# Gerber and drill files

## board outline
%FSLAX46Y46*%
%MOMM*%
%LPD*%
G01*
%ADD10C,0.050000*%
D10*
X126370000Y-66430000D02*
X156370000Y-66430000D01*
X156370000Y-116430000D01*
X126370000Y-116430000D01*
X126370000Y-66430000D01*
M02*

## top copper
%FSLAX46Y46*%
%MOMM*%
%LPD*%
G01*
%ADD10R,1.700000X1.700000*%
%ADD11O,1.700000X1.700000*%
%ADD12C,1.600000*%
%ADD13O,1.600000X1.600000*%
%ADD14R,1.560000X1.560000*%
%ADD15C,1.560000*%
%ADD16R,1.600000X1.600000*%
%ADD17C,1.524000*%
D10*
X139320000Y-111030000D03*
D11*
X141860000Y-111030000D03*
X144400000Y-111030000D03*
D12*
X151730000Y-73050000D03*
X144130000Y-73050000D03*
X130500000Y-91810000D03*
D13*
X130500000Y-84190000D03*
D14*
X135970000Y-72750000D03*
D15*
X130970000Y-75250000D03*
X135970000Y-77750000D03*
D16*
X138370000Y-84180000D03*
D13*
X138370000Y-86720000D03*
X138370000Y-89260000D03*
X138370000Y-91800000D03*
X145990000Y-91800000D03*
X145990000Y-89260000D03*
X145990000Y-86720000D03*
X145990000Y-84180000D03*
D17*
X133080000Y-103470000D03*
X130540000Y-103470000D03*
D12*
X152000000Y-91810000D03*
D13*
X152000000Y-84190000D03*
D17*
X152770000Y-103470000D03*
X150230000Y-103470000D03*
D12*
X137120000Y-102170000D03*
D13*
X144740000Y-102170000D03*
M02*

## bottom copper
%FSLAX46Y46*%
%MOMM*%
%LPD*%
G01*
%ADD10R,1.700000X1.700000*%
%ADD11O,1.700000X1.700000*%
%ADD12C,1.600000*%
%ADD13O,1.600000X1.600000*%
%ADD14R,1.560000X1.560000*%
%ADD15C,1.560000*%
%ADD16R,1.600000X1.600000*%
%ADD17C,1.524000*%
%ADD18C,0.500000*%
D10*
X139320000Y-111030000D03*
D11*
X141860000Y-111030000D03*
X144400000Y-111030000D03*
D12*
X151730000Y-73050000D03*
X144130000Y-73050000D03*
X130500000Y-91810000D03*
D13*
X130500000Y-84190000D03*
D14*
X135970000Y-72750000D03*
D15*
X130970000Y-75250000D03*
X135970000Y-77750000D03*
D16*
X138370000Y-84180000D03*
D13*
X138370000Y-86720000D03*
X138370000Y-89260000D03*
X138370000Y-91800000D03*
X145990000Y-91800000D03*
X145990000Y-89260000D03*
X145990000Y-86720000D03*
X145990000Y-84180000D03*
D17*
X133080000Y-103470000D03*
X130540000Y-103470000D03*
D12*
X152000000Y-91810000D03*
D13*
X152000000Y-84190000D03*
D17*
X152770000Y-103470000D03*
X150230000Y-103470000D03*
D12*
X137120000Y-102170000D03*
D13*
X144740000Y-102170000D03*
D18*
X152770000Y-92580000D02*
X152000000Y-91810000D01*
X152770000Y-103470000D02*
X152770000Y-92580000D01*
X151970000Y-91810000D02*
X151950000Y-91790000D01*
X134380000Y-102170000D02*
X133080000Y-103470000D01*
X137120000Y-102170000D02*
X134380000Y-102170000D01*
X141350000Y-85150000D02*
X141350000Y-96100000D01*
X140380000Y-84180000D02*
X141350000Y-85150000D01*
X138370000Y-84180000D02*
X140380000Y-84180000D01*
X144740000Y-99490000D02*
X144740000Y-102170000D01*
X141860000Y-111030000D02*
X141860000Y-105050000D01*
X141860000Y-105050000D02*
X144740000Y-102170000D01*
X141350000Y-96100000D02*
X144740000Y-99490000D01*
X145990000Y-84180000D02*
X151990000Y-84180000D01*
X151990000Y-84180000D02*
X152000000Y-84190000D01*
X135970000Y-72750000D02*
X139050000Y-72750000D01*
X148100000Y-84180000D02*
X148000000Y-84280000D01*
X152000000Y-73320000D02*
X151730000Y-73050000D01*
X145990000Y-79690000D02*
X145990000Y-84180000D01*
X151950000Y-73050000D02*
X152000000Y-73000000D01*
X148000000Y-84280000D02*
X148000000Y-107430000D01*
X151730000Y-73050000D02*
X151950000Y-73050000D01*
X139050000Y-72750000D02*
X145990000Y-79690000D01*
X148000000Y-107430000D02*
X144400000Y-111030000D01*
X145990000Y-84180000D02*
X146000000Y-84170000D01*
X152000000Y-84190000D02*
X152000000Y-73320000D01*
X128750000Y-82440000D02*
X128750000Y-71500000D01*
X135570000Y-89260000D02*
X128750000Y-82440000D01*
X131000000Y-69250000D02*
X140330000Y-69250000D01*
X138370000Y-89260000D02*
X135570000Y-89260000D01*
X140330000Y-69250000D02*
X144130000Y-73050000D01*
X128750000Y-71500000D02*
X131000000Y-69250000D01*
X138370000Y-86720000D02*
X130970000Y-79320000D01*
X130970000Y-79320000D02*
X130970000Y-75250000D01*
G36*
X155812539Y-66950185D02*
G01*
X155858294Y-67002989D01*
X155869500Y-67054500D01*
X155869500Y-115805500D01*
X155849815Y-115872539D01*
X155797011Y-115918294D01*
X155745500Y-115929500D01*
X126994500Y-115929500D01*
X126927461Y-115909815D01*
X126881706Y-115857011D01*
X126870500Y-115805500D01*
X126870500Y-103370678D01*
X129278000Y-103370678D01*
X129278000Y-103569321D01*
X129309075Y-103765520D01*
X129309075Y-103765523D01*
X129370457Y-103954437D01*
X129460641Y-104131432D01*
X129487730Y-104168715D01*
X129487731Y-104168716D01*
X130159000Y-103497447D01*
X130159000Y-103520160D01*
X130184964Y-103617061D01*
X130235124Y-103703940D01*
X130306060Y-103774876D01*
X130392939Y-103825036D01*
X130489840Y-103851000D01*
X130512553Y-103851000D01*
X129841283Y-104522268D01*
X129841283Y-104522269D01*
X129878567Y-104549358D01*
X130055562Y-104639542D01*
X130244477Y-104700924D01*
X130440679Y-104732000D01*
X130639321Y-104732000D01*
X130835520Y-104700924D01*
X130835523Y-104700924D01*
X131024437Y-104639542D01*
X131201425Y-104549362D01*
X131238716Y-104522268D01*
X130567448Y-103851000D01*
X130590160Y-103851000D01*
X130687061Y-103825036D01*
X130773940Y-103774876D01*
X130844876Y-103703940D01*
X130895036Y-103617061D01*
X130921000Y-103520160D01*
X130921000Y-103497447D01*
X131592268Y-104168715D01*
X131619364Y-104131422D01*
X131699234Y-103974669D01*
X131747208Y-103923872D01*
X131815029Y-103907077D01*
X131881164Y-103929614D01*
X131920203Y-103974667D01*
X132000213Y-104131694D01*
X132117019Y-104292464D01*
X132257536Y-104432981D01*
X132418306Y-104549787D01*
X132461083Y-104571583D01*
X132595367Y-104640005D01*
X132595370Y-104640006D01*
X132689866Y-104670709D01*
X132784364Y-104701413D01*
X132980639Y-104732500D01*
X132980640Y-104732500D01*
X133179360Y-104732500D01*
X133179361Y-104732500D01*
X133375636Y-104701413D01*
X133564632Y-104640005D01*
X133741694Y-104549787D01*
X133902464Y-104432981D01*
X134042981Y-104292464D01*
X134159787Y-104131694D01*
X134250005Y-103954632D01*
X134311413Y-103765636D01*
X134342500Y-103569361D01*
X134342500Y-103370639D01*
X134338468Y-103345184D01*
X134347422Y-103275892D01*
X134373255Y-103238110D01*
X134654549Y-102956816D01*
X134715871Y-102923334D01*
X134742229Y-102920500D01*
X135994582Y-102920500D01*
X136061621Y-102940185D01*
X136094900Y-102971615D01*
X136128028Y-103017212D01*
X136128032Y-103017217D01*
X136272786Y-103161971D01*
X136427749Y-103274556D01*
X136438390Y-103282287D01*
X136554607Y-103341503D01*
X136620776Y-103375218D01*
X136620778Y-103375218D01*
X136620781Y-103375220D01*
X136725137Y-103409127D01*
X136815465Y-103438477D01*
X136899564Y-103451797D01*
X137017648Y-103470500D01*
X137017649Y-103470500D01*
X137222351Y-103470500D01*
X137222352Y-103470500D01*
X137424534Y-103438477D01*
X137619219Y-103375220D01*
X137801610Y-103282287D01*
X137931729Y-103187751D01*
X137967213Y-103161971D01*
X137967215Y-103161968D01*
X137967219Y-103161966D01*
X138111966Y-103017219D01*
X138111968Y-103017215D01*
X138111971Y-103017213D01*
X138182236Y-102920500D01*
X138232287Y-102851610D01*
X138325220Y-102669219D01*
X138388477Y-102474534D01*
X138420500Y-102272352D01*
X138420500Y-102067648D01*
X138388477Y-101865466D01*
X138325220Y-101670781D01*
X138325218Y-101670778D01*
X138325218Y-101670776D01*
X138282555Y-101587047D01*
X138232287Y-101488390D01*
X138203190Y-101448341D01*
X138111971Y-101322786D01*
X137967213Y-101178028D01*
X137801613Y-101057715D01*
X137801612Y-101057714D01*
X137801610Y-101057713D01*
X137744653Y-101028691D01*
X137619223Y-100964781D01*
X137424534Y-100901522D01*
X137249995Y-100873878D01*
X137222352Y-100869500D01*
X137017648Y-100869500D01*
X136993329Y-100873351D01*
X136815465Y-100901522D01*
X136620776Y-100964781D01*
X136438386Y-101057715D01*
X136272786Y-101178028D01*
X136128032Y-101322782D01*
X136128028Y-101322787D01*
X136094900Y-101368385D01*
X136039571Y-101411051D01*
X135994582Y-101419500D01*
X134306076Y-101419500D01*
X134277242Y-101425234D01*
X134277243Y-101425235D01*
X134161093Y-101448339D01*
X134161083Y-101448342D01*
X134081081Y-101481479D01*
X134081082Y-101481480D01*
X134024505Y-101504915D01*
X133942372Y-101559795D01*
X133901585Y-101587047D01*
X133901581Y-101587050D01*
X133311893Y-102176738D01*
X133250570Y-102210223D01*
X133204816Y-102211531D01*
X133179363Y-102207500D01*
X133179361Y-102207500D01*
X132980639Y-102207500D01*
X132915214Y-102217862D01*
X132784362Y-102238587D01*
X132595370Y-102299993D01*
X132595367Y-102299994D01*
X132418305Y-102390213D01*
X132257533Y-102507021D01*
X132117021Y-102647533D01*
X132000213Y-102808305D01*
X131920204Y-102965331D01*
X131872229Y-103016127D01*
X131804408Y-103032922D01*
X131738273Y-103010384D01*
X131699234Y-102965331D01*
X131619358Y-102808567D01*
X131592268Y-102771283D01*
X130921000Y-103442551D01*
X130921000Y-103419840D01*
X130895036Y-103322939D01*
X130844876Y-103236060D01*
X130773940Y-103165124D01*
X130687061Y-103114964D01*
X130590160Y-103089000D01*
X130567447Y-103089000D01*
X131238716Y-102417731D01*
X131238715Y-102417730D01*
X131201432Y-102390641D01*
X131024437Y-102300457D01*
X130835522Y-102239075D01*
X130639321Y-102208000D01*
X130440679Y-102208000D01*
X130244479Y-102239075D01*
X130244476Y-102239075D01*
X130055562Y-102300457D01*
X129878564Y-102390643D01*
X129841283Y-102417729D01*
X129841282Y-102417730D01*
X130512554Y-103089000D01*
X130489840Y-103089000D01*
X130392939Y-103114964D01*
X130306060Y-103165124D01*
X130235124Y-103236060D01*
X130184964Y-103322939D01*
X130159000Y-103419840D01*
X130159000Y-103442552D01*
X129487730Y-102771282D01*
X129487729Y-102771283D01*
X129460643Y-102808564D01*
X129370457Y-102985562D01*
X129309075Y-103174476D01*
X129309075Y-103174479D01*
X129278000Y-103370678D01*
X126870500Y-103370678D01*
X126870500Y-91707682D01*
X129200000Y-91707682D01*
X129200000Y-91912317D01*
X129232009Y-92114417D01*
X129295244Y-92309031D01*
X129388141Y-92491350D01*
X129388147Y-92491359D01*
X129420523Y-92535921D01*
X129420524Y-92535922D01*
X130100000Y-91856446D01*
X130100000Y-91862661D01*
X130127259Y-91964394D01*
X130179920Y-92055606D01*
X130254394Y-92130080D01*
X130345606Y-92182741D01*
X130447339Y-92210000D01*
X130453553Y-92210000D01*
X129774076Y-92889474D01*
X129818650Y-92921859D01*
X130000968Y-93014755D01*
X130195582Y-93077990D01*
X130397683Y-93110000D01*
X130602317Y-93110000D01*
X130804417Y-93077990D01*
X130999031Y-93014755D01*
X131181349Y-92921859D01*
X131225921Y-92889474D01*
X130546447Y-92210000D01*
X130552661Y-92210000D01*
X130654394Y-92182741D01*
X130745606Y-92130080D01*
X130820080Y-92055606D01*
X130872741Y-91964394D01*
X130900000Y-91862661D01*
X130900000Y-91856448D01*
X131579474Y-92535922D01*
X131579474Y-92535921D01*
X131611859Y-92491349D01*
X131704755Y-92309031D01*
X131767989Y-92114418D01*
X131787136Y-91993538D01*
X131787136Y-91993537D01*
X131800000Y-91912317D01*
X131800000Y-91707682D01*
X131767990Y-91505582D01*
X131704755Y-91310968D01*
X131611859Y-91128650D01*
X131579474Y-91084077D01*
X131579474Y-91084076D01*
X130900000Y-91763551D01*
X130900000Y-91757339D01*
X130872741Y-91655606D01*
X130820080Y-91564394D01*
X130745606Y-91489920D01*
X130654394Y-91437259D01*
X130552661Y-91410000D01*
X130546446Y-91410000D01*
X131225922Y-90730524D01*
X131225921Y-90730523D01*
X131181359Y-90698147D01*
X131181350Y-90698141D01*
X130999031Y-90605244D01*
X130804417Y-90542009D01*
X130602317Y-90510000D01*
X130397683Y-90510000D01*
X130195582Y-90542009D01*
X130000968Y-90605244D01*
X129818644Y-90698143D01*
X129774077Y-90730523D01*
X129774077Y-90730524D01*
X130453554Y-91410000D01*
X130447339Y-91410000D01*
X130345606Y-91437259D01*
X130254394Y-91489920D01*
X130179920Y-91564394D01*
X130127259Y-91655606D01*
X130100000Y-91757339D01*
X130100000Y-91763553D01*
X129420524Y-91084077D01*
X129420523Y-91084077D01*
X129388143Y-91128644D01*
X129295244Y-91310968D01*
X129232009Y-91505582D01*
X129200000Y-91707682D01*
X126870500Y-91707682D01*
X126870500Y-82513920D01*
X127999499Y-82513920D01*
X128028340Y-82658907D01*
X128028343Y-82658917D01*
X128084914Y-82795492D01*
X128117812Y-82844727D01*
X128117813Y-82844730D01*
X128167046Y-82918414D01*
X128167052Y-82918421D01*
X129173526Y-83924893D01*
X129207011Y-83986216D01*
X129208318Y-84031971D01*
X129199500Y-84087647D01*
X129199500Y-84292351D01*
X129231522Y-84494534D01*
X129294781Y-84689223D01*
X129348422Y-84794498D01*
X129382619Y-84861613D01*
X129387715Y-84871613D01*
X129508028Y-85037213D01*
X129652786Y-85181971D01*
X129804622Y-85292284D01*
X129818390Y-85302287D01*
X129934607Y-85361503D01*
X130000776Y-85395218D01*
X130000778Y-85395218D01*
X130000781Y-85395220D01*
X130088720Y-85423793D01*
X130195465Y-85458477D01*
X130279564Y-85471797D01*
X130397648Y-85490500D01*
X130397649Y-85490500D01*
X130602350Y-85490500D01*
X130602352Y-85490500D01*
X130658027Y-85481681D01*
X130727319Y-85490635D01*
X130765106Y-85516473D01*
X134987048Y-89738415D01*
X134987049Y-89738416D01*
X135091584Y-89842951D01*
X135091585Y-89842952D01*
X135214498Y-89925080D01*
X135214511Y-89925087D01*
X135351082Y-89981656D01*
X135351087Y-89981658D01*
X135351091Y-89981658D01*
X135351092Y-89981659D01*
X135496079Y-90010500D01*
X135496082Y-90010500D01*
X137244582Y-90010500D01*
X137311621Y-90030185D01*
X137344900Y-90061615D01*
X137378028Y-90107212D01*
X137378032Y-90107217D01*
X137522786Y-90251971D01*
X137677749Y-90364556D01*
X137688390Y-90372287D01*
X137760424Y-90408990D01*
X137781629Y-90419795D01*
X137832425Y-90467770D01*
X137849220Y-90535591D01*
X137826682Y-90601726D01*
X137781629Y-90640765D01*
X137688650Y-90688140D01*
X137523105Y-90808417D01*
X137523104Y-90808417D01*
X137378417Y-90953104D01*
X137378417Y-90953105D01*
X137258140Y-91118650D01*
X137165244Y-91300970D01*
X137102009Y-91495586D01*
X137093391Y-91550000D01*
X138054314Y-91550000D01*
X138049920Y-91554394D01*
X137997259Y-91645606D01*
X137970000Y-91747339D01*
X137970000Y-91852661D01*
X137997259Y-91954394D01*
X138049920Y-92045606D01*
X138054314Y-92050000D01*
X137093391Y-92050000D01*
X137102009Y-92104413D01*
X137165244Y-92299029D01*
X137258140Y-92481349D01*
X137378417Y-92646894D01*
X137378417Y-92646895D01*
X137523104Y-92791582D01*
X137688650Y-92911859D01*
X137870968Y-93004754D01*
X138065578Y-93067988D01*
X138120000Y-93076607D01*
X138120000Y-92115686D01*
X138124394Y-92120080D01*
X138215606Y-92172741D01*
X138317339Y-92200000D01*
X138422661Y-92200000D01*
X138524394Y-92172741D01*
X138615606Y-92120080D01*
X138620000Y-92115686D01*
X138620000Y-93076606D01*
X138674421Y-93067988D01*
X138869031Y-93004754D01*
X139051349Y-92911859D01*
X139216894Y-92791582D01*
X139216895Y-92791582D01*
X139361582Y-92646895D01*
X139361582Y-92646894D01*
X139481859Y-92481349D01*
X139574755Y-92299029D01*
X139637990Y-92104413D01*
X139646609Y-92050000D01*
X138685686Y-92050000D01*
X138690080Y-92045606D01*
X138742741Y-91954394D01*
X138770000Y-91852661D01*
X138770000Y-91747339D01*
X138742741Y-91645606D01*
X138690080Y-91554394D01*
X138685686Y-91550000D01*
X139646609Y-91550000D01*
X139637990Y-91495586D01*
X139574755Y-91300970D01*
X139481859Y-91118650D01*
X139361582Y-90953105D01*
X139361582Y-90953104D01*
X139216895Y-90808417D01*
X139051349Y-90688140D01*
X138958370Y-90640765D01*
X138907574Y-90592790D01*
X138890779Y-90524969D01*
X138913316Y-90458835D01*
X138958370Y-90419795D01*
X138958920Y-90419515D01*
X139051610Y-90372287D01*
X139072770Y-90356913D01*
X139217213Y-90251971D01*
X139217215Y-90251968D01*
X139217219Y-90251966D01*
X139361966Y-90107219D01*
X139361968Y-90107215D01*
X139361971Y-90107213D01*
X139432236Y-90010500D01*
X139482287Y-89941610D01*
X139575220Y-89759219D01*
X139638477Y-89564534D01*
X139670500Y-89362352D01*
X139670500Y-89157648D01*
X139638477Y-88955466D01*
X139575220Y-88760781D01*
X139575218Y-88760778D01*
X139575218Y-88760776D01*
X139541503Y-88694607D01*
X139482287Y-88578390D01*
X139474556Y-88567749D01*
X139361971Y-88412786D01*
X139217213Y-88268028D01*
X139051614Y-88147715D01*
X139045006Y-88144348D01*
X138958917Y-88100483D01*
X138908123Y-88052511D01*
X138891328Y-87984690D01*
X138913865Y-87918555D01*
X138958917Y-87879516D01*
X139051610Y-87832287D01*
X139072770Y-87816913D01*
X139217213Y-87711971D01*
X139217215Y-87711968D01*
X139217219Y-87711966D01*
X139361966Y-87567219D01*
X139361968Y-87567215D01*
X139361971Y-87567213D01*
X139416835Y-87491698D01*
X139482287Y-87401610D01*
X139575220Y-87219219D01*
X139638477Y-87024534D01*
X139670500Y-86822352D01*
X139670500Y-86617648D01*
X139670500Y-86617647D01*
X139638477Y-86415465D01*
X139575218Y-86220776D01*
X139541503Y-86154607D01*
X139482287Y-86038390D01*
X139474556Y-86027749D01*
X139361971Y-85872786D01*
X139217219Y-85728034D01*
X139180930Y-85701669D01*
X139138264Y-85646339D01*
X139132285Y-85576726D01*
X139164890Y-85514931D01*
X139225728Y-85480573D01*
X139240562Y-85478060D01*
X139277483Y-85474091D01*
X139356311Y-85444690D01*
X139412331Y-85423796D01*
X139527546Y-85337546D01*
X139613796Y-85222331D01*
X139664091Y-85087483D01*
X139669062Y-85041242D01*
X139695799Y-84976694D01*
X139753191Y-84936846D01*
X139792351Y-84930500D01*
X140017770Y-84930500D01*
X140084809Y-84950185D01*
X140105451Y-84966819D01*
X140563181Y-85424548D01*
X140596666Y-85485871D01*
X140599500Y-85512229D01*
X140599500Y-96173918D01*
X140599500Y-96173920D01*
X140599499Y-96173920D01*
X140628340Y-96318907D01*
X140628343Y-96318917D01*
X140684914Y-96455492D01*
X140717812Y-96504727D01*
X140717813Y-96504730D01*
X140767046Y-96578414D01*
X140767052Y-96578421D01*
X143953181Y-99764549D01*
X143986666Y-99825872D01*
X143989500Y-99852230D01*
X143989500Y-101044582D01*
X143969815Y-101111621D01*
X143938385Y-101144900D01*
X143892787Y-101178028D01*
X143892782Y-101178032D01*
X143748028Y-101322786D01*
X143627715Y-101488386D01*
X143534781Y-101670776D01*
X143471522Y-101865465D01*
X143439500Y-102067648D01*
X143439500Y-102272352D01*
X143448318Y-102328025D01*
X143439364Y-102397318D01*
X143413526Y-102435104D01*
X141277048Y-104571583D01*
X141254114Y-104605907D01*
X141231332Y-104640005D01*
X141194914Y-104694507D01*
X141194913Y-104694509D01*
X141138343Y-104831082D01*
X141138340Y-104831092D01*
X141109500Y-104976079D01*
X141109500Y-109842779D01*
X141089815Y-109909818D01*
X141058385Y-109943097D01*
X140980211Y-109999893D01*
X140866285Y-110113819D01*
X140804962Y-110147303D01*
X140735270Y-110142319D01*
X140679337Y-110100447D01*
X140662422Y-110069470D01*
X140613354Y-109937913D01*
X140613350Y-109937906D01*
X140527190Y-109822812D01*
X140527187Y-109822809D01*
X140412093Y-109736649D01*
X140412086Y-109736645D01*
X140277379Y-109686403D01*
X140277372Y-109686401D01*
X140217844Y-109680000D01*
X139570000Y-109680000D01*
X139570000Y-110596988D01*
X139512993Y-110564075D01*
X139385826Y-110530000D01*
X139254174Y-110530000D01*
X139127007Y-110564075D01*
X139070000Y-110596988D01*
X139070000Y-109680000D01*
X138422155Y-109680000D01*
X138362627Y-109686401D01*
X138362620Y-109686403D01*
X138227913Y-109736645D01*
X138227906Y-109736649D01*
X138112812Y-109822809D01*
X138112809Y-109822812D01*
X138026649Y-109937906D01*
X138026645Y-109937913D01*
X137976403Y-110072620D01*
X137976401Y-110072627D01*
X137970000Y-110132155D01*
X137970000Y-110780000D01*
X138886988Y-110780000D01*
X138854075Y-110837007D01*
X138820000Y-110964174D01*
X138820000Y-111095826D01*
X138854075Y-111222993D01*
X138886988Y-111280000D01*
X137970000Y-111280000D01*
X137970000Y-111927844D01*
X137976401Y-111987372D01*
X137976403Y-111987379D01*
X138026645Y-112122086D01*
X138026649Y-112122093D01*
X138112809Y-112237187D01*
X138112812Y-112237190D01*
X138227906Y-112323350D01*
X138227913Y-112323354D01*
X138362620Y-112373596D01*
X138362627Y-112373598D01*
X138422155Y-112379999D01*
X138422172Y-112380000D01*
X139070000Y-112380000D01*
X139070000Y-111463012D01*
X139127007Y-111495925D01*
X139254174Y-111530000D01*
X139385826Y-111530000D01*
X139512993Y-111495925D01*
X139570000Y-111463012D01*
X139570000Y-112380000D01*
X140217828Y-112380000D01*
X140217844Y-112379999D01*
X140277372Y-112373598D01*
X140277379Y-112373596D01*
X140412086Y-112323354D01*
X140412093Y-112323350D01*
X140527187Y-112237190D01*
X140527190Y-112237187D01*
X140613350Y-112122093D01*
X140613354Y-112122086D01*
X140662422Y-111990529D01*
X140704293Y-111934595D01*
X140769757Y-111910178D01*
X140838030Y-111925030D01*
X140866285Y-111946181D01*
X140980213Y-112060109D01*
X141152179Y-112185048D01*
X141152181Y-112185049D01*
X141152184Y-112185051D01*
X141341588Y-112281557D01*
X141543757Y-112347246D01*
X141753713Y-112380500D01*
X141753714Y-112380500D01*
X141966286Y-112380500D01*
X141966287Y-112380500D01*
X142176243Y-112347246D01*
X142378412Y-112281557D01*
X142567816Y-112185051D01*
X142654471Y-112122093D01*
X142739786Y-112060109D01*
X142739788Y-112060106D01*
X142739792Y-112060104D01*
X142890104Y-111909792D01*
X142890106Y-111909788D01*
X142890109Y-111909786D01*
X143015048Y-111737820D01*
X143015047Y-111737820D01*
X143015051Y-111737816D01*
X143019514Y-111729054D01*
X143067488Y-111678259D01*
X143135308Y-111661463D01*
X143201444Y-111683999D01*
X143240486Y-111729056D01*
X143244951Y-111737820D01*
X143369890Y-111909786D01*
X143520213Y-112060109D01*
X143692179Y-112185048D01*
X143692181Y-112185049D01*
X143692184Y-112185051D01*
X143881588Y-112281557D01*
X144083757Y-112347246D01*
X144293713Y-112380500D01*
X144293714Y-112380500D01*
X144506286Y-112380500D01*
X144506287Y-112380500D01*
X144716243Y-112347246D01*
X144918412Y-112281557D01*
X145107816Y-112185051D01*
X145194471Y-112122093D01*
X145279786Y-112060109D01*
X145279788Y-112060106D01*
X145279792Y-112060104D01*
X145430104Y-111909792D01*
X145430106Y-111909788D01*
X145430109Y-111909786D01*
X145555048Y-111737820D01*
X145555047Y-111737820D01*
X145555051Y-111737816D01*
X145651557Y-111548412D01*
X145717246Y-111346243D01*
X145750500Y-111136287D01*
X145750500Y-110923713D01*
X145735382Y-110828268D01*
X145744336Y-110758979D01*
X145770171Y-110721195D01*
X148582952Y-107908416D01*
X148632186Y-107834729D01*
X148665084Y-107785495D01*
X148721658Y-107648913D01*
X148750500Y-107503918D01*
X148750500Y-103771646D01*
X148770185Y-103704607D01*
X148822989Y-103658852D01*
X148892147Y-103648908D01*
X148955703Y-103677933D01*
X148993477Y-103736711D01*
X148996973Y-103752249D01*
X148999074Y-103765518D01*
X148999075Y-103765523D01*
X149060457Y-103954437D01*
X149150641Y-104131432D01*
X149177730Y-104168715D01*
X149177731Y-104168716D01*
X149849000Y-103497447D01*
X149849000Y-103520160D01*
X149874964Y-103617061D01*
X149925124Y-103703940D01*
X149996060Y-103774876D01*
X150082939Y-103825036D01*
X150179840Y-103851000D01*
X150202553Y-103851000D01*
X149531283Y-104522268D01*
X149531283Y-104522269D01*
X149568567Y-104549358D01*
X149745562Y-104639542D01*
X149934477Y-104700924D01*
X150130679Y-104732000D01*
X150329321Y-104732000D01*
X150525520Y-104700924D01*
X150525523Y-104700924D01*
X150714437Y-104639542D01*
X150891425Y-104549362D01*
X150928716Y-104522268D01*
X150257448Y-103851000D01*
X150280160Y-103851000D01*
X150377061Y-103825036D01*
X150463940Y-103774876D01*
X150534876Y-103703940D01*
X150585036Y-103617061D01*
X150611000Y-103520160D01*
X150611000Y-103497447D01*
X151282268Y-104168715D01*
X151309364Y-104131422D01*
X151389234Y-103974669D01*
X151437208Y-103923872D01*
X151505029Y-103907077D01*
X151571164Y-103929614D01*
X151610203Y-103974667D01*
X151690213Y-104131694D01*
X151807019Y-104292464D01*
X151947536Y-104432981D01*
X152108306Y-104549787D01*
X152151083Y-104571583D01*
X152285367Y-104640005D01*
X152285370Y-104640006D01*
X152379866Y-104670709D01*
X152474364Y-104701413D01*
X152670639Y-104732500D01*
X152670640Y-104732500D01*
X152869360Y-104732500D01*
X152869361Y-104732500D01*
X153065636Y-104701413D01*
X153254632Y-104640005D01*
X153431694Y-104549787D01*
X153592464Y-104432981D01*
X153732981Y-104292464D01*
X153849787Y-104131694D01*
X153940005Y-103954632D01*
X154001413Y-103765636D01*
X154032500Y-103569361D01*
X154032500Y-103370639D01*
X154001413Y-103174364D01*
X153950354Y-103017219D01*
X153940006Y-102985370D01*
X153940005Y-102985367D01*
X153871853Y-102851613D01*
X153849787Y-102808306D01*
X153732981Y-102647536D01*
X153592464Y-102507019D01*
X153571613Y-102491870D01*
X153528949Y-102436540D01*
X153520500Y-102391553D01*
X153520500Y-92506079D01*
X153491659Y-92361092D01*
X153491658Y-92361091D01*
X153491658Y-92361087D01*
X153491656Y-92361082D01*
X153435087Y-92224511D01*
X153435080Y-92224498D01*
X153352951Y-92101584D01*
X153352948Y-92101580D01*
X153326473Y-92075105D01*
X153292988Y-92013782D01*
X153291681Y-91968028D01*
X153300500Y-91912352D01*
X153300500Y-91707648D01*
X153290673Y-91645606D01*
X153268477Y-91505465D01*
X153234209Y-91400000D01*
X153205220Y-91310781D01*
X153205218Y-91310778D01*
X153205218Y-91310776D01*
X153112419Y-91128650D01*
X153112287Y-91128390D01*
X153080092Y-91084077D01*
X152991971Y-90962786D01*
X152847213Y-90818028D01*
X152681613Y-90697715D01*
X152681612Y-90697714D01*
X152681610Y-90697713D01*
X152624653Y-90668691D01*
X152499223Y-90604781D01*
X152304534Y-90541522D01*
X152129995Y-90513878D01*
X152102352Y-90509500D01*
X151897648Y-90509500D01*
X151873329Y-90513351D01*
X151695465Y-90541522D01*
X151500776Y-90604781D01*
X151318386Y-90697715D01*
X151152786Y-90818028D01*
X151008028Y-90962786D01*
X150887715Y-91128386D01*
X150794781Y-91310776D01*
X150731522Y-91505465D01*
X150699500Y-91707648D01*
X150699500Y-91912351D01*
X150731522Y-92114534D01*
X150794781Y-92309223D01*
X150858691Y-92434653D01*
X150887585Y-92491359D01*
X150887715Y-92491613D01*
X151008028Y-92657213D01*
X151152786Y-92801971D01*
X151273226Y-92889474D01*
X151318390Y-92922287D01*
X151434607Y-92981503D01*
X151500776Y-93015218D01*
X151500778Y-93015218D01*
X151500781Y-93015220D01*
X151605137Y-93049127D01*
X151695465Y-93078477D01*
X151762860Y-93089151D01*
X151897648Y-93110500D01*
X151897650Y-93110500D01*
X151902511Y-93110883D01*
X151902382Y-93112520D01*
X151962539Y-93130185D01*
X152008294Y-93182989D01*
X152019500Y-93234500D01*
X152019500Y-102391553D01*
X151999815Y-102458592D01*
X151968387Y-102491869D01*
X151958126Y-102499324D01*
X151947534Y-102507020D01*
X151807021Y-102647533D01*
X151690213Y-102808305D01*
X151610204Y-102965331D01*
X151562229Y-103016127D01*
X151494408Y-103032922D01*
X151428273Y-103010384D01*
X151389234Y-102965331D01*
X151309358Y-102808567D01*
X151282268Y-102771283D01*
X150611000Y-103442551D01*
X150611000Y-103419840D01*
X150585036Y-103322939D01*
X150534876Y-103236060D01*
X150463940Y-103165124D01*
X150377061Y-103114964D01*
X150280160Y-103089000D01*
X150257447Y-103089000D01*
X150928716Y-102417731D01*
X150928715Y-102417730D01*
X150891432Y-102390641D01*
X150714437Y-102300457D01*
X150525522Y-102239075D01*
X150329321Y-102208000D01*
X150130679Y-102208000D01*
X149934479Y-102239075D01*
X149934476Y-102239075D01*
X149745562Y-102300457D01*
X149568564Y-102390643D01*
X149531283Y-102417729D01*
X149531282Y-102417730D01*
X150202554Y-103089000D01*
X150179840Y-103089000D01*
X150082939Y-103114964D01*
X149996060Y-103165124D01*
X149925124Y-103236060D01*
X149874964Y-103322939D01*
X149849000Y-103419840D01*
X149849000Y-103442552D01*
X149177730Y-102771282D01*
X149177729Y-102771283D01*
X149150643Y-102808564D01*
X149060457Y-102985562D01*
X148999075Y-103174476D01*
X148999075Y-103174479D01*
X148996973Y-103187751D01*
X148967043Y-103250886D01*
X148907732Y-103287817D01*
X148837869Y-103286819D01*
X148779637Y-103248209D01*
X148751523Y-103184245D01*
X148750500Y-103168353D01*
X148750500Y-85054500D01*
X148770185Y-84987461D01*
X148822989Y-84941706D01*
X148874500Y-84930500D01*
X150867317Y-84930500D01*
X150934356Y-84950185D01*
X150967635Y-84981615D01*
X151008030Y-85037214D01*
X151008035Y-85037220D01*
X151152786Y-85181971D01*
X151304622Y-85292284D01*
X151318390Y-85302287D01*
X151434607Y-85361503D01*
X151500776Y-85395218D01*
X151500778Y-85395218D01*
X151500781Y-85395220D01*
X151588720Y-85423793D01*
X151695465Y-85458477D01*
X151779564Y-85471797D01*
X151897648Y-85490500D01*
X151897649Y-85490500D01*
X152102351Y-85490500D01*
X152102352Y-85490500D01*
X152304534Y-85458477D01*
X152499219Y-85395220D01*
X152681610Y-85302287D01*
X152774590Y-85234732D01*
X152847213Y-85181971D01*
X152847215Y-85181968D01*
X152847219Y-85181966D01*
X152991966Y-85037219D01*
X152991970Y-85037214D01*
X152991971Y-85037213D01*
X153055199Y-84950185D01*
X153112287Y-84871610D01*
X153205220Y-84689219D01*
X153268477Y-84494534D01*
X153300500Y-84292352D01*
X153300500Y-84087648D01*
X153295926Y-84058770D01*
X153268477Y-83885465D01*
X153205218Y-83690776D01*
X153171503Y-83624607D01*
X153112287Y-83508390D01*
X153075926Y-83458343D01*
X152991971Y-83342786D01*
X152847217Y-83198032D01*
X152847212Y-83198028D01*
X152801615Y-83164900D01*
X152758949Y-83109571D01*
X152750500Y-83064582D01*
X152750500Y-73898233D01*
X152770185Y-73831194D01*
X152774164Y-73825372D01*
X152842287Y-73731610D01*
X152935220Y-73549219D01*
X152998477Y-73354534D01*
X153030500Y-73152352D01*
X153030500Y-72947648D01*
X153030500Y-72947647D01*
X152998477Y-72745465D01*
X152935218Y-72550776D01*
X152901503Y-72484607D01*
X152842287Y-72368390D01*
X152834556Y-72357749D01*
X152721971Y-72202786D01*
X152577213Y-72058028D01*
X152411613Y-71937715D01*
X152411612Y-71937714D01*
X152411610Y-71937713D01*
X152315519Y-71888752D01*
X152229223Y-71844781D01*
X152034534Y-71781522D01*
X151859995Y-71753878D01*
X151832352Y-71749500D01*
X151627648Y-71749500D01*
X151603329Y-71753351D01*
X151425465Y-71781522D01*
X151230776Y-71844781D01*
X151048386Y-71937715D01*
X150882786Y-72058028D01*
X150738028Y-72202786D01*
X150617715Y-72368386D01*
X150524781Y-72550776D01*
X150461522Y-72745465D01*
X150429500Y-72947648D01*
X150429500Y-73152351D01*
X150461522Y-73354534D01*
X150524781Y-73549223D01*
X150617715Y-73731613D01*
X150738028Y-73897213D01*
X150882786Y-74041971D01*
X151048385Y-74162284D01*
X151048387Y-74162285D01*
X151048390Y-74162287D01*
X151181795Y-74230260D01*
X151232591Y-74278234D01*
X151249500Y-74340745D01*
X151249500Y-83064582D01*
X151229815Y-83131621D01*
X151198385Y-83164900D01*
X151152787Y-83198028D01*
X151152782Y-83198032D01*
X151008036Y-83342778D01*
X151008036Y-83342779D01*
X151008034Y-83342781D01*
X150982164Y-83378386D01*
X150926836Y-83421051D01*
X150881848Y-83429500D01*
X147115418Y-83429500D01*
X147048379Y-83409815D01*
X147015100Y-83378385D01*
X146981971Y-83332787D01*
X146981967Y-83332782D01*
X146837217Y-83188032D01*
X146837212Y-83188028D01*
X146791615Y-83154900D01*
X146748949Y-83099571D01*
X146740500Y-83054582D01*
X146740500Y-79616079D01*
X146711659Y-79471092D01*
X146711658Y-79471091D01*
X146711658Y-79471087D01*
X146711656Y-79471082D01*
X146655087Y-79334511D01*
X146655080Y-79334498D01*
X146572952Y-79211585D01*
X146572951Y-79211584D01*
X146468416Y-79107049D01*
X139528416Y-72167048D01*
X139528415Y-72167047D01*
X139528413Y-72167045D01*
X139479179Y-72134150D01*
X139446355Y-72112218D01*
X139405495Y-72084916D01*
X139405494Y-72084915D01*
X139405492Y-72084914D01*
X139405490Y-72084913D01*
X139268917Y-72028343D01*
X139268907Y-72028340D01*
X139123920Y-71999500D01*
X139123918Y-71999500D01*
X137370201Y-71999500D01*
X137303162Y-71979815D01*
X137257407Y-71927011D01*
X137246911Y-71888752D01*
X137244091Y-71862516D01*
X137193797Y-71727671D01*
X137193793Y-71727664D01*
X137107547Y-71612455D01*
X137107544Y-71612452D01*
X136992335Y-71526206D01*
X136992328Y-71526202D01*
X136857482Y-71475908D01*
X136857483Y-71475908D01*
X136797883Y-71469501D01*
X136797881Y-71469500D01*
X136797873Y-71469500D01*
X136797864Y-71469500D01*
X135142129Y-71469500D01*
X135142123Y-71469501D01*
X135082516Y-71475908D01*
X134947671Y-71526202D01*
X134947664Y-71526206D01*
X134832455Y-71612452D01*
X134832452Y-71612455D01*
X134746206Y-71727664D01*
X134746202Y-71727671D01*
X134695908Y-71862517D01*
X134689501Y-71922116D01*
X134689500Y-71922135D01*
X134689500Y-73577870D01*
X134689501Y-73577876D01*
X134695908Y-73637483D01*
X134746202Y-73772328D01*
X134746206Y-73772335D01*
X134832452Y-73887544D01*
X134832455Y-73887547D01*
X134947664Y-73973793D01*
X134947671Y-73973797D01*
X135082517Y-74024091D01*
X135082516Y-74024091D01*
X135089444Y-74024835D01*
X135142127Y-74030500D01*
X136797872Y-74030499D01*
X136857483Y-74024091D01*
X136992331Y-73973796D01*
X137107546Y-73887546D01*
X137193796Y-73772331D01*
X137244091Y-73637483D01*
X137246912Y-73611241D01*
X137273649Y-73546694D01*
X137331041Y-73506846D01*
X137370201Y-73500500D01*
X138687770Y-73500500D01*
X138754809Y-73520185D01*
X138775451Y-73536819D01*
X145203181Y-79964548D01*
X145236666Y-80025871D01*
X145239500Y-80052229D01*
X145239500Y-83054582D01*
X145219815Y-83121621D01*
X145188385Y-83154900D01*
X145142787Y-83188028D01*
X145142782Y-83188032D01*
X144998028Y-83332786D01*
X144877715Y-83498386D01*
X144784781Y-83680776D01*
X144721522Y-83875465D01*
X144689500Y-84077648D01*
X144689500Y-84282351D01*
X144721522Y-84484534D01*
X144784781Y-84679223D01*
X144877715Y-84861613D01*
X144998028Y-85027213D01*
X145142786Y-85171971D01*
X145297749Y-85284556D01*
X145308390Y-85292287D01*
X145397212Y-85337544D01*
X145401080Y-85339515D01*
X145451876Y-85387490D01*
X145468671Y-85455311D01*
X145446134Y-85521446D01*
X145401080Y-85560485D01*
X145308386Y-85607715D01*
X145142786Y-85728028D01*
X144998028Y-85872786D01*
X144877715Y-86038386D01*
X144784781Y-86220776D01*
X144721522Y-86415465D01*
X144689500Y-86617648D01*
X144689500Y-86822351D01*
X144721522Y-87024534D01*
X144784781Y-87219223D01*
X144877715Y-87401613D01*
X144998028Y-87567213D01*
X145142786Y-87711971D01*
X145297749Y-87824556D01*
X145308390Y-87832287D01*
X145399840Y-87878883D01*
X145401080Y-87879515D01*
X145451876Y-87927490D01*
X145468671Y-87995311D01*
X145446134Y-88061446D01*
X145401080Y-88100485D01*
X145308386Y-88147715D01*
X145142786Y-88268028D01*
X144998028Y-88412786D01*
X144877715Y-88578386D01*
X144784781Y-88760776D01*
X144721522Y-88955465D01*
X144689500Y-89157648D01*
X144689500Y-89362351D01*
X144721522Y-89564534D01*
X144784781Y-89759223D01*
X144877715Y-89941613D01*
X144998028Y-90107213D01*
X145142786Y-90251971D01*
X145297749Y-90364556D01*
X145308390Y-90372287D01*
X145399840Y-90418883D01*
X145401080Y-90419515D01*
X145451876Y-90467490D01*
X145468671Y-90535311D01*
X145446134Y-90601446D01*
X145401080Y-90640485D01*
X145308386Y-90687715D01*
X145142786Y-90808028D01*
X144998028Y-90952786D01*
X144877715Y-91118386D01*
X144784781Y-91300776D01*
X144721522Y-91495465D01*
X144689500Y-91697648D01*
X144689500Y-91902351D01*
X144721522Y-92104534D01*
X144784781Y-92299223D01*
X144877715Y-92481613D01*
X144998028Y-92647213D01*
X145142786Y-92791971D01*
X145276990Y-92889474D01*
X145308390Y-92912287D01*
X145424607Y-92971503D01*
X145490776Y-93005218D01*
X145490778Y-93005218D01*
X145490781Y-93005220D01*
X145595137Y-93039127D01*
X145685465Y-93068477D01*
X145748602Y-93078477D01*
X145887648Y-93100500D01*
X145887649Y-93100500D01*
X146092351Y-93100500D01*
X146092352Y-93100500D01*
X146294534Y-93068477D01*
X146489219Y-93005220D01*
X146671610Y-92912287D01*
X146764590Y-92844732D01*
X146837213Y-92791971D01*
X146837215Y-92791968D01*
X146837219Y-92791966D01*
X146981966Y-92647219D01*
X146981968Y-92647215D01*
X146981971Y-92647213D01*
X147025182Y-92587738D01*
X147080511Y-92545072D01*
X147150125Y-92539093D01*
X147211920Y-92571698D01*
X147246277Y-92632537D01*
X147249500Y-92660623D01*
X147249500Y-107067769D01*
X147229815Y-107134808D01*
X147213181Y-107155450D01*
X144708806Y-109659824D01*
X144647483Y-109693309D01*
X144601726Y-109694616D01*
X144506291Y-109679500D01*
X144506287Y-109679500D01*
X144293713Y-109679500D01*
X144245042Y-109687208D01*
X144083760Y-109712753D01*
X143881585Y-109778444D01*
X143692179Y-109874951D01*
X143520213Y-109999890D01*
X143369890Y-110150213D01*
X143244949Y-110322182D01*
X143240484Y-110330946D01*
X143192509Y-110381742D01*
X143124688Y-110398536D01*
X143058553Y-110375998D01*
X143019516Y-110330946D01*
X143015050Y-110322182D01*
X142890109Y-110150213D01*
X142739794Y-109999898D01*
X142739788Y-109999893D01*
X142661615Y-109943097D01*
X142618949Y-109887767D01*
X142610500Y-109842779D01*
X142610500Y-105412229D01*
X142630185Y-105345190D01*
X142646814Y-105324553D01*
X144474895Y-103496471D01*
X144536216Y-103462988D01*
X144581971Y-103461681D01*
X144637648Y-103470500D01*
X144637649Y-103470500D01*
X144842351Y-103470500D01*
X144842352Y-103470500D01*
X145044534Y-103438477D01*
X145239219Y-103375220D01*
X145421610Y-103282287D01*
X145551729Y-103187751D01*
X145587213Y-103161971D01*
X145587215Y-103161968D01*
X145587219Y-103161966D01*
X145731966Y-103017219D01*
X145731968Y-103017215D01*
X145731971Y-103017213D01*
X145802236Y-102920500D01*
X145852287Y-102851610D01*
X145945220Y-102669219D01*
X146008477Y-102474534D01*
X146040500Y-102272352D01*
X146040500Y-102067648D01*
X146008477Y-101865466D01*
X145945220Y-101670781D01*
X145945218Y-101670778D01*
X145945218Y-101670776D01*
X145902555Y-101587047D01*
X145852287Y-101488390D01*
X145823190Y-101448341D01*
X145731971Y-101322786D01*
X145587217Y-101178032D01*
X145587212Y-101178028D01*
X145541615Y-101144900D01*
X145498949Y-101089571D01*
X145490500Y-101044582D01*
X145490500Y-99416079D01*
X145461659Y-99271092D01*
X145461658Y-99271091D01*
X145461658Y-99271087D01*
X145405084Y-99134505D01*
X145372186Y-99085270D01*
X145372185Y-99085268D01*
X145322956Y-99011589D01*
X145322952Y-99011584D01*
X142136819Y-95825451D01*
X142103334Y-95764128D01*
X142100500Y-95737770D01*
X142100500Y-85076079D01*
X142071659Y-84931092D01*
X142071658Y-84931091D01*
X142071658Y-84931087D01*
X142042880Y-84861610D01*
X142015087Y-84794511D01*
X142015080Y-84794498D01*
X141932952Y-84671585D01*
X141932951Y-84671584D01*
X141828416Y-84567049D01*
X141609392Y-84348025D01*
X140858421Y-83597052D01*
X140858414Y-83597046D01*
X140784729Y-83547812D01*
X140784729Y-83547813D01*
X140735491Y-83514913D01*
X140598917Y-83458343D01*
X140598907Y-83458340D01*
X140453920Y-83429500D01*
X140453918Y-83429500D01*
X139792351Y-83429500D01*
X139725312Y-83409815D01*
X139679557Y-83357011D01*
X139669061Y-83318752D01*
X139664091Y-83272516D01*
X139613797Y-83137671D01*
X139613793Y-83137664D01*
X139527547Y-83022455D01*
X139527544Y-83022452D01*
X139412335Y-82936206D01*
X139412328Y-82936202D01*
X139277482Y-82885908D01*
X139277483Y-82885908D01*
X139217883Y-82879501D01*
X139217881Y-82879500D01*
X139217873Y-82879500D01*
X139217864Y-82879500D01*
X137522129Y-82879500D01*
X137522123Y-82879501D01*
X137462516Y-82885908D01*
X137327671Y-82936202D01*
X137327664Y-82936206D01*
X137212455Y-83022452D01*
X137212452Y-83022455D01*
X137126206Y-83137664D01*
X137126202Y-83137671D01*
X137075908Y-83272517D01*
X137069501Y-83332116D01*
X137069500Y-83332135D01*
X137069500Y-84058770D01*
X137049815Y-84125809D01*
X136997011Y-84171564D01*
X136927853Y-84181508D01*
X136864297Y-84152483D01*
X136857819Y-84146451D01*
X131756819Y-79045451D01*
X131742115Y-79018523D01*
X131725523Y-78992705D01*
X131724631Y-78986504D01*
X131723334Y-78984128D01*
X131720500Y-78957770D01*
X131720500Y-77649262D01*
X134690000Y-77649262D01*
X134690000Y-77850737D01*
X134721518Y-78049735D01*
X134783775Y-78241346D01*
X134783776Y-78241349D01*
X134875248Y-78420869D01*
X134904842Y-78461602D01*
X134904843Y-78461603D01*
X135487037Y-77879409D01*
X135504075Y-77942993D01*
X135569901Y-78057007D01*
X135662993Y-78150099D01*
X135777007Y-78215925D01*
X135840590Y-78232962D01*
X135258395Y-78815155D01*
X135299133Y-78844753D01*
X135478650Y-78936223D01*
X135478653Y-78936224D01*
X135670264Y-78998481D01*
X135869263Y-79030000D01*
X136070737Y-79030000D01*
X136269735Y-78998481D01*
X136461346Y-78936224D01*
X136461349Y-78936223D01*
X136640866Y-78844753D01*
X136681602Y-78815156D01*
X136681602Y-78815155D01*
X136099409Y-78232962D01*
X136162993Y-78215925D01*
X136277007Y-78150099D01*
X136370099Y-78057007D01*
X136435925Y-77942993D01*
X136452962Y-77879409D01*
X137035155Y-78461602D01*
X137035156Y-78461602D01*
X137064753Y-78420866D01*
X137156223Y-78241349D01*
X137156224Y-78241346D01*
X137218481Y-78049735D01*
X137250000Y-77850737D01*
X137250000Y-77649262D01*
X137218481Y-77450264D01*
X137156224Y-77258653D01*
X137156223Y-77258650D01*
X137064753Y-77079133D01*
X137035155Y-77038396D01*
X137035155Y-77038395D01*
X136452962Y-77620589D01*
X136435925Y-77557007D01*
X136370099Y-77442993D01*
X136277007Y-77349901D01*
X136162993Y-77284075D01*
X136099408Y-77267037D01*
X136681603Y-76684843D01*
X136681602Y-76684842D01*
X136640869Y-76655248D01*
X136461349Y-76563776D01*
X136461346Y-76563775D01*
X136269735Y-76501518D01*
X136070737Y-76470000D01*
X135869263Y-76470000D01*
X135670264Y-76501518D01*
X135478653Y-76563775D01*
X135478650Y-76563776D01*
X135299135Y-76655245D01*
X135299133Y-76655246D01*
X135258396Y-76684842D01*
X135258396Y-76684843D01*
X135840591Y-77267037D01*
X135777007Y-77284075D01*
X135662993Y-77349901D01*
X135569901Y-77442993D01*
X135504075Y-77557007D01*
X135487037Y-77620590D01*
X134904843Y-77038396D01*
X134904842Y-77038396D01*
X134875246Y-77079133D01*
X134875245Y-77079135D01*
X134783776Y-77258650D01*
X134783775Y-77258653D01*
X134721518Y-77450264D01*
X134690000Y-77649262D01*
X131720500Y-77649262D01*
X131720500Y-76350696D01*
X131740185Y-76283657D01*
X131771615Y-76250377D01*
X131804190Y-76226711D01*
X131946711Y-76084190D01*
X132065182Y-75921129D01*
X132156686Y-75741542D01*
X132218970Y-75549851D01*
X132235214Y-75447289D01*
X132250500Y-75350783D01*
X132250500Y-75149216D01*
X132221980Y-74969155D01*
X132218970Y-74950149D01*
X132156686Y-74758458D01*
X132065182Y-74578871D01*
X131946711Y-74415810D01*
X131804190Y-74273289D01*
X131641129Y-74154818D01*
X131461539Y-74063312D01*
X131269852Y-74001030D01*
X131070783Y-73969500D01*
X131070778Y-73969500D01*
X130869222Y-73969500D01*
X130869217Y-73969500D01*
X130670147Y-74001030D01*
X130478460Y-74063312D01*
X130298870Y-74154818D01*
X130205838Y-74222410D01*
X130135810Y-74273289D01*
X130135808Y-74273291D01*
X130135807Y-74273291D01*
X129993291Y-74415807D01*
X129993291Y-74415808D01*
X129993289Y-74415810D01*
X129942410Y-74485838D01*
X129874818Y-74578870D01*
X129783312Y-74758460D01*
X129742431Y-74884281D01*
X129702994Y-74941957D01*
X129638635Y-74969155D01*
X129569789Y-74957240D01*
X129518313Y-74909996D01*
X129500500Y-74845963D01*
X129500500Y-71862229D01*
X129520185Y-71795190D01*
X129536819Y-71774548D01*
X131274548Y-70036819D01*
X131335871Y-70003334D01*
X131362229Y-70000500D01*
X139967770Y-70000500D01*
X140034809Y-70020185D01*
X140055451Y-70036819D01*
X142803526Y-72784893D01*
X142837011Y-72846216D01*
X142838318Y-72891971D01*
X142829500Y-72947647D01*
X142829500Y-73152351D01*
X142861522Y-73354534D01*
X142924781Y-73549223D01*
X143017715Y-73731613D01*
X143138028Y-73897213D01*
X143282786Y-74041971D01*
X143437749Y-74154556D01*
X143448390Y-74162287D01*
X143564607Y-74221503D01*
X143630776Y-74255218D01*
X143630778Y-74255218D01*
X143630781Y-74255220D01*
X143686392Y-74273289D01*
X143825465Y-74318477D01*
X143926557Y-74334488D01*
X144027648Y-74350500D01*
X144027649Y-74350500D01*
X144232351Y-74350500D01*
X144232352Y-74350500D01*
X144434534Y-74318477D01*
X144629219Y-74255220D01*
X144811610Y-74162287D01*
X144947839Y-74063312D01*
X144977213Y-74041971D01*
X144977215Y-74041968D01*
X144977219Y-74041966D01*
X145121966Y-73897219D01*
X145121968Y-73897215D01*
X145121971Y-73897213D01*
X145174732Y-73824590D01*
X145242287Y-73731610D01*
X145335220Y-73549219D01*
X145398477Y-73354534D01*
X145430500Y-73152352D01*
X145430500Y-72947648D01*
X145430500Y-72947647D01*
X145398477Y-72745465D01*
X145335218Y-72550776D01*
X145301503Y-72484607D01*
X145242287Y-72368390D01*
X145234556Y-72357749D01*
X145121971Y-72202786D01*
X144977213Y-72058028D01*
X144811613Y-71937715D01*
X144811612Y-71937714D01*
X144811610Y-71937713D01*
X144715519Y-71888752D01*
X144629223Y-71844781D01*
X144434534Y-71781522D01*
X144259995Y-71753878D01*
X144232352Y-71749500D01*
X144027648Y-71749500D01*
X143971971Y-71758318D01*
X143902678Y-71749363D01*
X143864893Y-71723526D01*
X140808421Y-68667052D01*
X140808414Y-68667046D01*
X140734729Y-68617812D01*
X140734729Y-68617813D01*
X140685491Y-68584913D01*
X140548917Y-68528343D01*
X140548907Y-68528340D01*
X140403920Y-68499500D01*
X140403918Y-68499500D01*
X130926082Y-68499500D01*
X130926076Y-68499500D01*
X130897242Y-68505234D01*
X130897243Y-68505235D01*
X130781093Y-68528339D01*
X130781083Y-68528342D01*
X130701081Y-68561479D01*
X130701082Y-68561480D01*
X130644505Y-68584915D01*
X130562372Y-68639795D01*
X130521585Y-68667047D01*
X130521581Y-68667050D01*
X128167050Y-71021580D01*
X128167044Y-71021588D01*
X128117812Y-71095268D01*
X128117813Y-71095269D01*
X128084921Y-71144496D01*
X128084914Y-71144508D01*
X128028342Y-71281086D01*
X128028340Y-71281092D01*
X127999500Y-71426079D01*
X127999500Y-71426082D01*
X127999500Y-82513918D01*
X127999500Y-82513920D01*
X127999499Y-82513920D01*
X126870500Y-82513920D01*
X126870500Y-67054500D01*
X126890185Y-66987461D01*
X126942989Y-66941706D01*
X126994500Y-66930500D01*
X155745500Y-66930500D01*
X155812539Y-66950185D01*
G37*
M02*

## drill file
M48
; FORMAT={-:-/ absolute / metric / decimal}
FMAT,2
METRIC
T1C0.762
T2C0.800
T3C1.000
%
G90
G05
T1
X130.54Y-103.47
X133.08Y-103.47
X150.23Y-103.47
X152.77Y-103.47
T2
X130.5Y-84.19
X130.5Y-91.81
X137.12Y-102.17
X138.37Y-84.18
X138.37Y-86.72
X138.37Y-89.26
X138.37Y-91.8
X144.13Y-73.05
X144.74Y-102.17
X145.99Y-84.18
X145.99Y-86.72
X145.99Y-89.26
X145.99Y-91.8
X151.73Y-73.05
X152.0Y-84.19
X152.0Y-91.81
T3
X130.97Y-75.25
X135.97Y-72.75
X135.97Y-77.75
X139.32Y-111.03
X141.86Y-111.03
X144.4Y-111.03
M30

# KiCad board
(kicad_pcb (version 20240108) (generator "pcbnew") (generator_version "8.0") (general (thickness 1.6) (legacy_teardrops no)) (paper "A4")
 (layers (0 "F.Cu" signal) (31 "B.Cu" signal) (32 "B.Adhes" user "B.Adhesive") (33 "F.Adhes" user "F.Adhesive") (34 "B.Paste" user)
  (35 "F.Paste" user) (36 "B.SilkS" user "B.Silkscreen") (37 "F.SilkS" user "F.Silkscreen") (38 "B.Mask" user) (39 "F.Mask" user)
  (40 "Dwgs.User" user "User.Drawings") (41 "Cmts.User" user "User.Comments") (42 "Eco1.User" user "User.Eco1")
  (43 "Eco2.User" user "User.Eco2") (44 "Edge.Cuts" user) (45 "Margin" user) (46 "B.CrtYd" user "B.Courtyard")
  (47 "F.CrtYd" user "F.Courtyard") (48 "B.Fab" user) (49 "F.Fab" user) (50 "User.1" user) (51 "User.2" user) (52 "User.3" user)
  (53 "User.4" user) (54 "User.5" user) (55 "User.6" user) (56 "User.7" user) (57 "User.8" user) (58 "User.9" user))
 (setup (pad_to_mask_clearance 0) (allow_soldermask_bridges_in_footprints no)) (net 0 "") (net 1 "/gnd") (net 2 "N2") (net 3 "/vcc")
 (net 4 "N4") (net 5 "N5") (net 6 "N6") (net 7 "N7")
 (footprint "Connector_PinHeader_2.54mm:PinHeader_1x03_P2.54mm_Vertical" (layer "F.Cu") (at 139.32 111.03 90)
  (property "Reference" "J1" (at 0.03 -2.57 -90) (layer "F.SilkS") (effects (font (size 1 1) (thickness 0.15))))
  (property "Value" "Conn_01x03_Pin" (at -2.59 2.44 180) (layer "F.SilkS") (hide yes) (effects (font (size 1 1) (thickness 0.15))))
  (pad "1" thru_hole rect (at 0 0 90) (size 1.7 1.7) (drill 1) (layers "*.Cu" "*.Mask") (remove_unused_layers no) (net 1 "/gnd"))
  (pad "2" thru_hole oval (at 0 2.54 90) (size 1.7 1.7) (drill 1) (layers "*.Cu" "*.Mask") (remove_unused_layers no) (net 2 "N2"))
  (pad "3" thru_hole oval (at 0 5.08 90) (size 1.7 1.7) (drill 1) (layers "*.Cu" "*.Mask") (remove_unused_layers no) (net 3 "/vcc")))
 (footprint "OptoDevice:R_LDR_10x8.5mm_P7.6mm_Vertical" (layer "F.Cu") (at 151.73 73.05 180)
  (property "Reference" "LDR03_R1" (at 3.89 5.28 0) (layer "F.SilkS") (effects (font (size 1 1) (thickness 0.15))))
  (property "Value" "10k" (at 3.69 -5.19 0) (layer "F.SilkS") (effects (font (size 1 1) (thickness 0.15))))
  (pad "1" thru_hole circle (at 0 0 180) (size 1.6 1.6) (drill 0.8) (layers "*.Cu" "*.Mask") (remove_unused_layers no) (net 3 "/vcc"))
  (pad "2" thru_hole circle (at 7.6 0 180) (size 1.6 1.6) (drill 0.8) (layers "*.Cu" "*.Mask") (remove_unused_layers no) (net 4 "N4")))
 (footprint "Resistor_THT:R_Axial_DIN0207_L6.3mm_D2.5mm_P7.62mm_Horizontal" (layer "F.Cu") (at 130.5 91.81 90)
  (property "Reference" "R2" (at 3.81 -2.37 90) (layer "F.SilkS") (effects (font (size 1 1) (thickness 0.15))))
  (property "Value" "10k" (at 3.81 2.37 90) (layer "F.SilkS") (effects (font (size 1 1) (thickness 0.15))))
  (pad "1" thru_hole circle (at 0 0 90) (size 1.6 1.6) (drill 0.8) (layers "*.Cu" "*.Mask") (remove_unused_layers no) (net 1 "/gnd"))
  (pad "2" thru_hole oval (at 7.62 0 90) (size 1.6 1.6) (drill 0.8) (layers "*.Cu" "*.Mask") (remove_unused_layers no) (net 4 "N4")))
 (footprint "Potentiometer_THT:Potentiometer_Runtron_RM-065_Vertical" (layer "F.Cu") (at 135.97 72.75 -90)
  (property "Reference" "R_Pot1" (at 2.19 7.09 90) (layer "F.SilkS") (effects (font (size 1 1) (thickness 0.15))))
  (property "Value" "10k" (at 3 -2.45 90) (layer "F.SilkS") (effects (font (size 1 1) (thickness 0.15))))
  (pad "1" thru_hole rect (at 0 0 270) (size 1.56 1.56) (drill 1) (layers "*.Cu" "*.Mask") (remove_unused_layers no) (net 3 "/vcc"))
  (pad "2" thru_hole circle (at 2.5 5 270) (size 1.56 1.56) (drill 1) (layers "*.Cu" "*.Mask") (remove_unused_layers no) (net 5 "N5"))
  (pad "3" thru_hole circle (at 5 0 270) (size 1.56 1.56) (drill 1) (layers "*.Cu" "*.Mask") (remove_unused_layers no) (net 1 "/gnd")))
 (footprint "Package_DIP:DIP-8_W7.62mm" (layer "F.Cu") (at 138.37 84.18)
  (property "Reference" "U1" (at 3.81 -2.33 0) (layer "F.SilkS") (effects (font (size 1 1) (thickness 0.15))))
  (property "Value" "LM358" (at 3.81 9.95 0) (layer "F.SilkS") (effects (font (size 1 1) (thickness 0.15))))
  (pad "1" thru_hole rect (at 0 0) (size 1.6 1.6) (drill 0.8) (layers "*.Cu" "*.Mask") (remove_unused_layers no) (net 2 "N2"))
  (pad "2" thru_hole oval (at 0 2.54) (size 1.6 1.6) (drill 0.8) (layers "*.Cu" "*.Mask") (remove_unused_layers no) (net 5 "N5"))
  (pad "3" thru_hole oval (at 0 5.08) (size 1.6 1.6) (drill 0.8) (layers "*.Cu" "*.Mask") (remove_unused_layers no) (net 4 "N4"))
  (pad "4" thru_hole oval (at 0 7.62) (size 1.6 1.6) (drill 0.8) (layers "*.Cu" "*.Mask") (remove_unused_layers no) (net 1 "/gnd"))
  (pad "5" thru_hole oval (at 7.62 7.62) (size 1.6 1.6) (drill 0.8) (layers "*.Cu" "*.Mask") (remove_unused_layers no))
  (pad "6" thru_hole oval (at 7.62 5.08) (size 1.6 1.6) (drill 0.8) (layers "*.Cu" "*.Mask") (remove_unused_layers no))
  (pad "7" thru_hole oval (at 7.62 2.54) (size 1.6 1.6) (drill 0.8) (layers "*.Cu" "*.Mask") (remove_unused_layers no))
  (pad "8" thru_hole oval (at 7.62 0) (size 1.6 1.6) (drill 0.8) (layers "*.Cu" "*.Mask") (remove_unused_layers no) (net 3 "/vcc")))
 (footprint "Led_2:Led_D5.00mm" (layer "F.Cu") (at 131.81 103.47 180)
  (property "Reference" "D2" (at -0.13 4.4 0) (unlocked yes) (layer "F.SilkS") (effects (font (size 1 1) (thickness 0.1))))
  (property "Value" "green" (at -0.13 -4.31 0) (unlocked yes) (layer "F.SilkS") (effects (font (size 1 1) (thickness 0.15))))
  (pad "1" thru_hole circle (at -1.27 0 180) (size 1.524 1.524) (drill 0.762) (layers "*.Cu" "*.Mask") (remove_unused_layers no)
   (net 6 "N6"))
  (pad "2" thru_hole circle (at 1.27 0 180) (size 1.524 1.524) (drill 0.762) (layers "*.Cu" "*.Mask") (remove_unused_layers no)
   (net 1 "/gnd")))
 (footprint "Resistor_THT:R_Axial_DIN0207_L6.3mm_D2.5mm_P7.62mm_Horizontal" (layer "F.Cu") (at 152 91.81 90)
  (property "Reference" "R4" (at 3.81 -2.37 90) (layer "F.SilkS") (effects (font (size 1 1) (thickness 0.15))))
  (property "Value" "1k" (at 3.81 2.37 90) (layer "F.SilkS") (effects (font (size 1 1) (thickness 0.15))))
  (pad "1" thru_hole circle (at 0 0 90) (size 1.6 1.6) (drill 0.8) (layers "*.Cu" "*.Mask") (remove_unused_layers no) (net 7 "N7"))
  (pad "2" thru_hole oval (at 7.62 0 90) (size 1.6 1.6) (drill 0.8) (layers "*.Cu" "*.Mask") (remove_unused_layers no) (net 3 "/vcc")))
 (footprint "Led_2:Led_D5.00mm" (layer "F.Cu") (at 151.5 103.47 180)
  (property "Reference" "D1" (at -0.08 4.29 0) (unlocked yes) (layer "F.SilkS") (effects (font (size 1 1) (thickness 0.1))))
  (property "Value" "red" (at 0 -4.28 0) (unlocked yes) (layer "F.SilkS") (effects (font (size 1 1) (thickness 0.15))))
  (pad "1" thru_hole circle (at -1.27 0 180) (size 1.524 1.524) (drill 0.762) (layers "*.Cu" "*.Mask") (remove_unused_layers no)
   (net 7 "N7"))
  (pad "2" thru_hole circle (at 1.27 0 180) (size 1.524 1.524) (drill 0.762) (layers "*.Cu" "*.Mask") (remove_unused_layers no)
   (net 1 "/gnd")))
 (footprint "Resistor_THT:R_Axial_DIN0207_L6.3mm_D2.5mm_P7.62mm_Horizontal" (layer "F.Cu") (at 137.12 102.17)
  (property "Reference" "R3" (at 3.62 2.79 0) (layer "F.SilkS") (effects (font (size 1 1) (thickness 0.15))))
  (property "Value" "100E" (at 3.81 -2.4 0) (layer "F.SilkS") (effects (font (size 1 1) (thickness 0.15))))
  (pad "1" thru_hole circle (at 0 0) (size 1.6 1.6) (drill 0.8) (layers "*.Cu" "*.Mask") (remove_unused_layers no) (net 6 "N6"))
  (pad "2" thru_hole oval (at 7.62 0) (size 1.6 1.6) (drill 0.8) (layers "*.Cu" "*.Mask") (remove_unused_layers no) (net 2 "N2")))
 (gr_rect (start 126.37 66.43) (end 156.37 116.43) (stroke (width 0.05) (type default)) (fill none) (layer "Edge.Cuts"))
 (segment (start 152.77 92.58) (end 152 91.81) (width 0.5) (layer "B.Cu") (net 7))
 (segment (start 152.77 103.47) (end 152.77 92.58) (width 0.5) (layer "B.Cu") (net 7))
 (segment (start 151.97 91.81) (end 151.95 91.79) (width 0.5) (layer "B.Cu") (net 7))
 (segment (start 134.38 102.17) (end 133.08 103.47) (width 0.5) (layer "B.Cu") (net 6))
 (segment (start 137.12 102.17) (end 134.38 102.17) (width 0.5) (layer "B.Cu") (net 6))
 (segment (start 141.35 85.15) (end 141.35 96.1) (width 0.5) (layer "B.Cu") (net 2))
 (segment (start 140.38 84.18) (end 141.35 85.15) (width 0.5) (layer "B.Cu") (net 2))
 (segment (start 138.37 84.18) (end 140.38 84.18) (width 0.5) (layer "B.Cu") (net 2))
 (segment (start 144.74 99.49) (end 144.74 102.17) (width 0.5) (layer "B.Cu") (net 2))
 (segment (start 141.86 111.03) (end 141.86 105.05) (width 0.5) (layer "B.Cu") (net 2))
 (segment (start 141.86 105.05) (end 144.74 102.17) (width 0.5) (layer "B.Cu") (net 2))
 (segment (start 141.35 96.1) (end 144.74 99.49) (width 0.5) (layer "B.Cu") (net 2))
 (segment (start 145.99 84.18) (end 151.99 84.18) (width 0.5) (layer "B.Cu") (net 3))
 (segment (start 151.99 84.18) (end 152 84.19) (width 0.5) (layer "B.Cu") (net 3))
 (segment (start 135.97 72.75) (end 139.05 72.75) (width 0.5) (layer "B.Cu") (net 3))
 (segment (start 148.1 84.18) (end 148 84.28) (width 0.5) (layer "B.Cu") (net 3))
 (segment (start 152 73.32) (end 151.73 73.05) (width 0.5) (layer "B.Cu") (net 3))
 (segment (start 145.99 79.69) (end 145.99 84.18) (width 0.5) (layer "B.Cu") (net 3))
 (segment (start 151.95 73.05) (end 152 73) (width 0.5) (layer "B.Cu") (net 3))
 (segment (start 148 84.28) (end 148 107.43) (width 0.5) (layer "B.Cu") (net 3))
 (segment (start 151.73 73.05) (end 151.95 73.05) (width 0.5) (layer "B.Cu") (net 3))
 (segment (start 139.05 72.75) (end 145.99 79.69) (width 0.5) (layer "B.Cu") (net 3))
 (segment (start 148 107.43) (end 144.4 111.03) (width 0.5) (layer "B.Cu") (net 3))
 (segment (start 145.99 84.18) (end 146 84.17) (width 0.5) (layer "B.Cu") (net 3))
 (segment (start 152 84.19) (end 152 73.32) (width 0.5) (layer "B.Cu") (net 3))
 (segment (start 128.75 82.44) (end 128.75 71.5) (width 0.5) (layer "B.Cu") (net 4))
 (segment (start 135.57 89.26) (end 128.75 82.44) (width 0.5) (layer "B.Cu") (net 4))
 (segment (start 131 69.25) (end 140.33 69.25) (width 0.5) (layer "B.Cu") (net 4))
 (segment (start 138.37 89.26) (end 135.57 89.26) (width 0.5) (layer "B.Cu") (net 4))
 (segment (start 140.33 69.25) (end 144.13 73.05) (width 0.5) (layer "B.Cu") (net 4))
 (segment (start 128.75 71.5) (end 131 69.25) (width 0.5) (layer "B.Cu") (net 4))
 (segment (start 138.37 86.72) (end 130.97 79.32) (width 0.5) (layer "B.Cu") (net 5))
 (segment (start 130.97 79.32) (end 130.97 75.25) (width 0.5) (layer "B.Cu") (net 5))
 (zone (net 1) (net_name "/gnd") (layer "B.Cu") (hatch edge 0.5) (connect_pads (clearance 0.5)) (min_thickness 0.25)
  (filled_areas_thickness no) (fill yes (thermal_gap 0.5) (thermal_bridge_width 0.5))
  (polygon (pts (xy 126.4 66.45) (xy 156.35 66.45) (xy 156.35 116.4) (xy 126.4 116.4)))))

